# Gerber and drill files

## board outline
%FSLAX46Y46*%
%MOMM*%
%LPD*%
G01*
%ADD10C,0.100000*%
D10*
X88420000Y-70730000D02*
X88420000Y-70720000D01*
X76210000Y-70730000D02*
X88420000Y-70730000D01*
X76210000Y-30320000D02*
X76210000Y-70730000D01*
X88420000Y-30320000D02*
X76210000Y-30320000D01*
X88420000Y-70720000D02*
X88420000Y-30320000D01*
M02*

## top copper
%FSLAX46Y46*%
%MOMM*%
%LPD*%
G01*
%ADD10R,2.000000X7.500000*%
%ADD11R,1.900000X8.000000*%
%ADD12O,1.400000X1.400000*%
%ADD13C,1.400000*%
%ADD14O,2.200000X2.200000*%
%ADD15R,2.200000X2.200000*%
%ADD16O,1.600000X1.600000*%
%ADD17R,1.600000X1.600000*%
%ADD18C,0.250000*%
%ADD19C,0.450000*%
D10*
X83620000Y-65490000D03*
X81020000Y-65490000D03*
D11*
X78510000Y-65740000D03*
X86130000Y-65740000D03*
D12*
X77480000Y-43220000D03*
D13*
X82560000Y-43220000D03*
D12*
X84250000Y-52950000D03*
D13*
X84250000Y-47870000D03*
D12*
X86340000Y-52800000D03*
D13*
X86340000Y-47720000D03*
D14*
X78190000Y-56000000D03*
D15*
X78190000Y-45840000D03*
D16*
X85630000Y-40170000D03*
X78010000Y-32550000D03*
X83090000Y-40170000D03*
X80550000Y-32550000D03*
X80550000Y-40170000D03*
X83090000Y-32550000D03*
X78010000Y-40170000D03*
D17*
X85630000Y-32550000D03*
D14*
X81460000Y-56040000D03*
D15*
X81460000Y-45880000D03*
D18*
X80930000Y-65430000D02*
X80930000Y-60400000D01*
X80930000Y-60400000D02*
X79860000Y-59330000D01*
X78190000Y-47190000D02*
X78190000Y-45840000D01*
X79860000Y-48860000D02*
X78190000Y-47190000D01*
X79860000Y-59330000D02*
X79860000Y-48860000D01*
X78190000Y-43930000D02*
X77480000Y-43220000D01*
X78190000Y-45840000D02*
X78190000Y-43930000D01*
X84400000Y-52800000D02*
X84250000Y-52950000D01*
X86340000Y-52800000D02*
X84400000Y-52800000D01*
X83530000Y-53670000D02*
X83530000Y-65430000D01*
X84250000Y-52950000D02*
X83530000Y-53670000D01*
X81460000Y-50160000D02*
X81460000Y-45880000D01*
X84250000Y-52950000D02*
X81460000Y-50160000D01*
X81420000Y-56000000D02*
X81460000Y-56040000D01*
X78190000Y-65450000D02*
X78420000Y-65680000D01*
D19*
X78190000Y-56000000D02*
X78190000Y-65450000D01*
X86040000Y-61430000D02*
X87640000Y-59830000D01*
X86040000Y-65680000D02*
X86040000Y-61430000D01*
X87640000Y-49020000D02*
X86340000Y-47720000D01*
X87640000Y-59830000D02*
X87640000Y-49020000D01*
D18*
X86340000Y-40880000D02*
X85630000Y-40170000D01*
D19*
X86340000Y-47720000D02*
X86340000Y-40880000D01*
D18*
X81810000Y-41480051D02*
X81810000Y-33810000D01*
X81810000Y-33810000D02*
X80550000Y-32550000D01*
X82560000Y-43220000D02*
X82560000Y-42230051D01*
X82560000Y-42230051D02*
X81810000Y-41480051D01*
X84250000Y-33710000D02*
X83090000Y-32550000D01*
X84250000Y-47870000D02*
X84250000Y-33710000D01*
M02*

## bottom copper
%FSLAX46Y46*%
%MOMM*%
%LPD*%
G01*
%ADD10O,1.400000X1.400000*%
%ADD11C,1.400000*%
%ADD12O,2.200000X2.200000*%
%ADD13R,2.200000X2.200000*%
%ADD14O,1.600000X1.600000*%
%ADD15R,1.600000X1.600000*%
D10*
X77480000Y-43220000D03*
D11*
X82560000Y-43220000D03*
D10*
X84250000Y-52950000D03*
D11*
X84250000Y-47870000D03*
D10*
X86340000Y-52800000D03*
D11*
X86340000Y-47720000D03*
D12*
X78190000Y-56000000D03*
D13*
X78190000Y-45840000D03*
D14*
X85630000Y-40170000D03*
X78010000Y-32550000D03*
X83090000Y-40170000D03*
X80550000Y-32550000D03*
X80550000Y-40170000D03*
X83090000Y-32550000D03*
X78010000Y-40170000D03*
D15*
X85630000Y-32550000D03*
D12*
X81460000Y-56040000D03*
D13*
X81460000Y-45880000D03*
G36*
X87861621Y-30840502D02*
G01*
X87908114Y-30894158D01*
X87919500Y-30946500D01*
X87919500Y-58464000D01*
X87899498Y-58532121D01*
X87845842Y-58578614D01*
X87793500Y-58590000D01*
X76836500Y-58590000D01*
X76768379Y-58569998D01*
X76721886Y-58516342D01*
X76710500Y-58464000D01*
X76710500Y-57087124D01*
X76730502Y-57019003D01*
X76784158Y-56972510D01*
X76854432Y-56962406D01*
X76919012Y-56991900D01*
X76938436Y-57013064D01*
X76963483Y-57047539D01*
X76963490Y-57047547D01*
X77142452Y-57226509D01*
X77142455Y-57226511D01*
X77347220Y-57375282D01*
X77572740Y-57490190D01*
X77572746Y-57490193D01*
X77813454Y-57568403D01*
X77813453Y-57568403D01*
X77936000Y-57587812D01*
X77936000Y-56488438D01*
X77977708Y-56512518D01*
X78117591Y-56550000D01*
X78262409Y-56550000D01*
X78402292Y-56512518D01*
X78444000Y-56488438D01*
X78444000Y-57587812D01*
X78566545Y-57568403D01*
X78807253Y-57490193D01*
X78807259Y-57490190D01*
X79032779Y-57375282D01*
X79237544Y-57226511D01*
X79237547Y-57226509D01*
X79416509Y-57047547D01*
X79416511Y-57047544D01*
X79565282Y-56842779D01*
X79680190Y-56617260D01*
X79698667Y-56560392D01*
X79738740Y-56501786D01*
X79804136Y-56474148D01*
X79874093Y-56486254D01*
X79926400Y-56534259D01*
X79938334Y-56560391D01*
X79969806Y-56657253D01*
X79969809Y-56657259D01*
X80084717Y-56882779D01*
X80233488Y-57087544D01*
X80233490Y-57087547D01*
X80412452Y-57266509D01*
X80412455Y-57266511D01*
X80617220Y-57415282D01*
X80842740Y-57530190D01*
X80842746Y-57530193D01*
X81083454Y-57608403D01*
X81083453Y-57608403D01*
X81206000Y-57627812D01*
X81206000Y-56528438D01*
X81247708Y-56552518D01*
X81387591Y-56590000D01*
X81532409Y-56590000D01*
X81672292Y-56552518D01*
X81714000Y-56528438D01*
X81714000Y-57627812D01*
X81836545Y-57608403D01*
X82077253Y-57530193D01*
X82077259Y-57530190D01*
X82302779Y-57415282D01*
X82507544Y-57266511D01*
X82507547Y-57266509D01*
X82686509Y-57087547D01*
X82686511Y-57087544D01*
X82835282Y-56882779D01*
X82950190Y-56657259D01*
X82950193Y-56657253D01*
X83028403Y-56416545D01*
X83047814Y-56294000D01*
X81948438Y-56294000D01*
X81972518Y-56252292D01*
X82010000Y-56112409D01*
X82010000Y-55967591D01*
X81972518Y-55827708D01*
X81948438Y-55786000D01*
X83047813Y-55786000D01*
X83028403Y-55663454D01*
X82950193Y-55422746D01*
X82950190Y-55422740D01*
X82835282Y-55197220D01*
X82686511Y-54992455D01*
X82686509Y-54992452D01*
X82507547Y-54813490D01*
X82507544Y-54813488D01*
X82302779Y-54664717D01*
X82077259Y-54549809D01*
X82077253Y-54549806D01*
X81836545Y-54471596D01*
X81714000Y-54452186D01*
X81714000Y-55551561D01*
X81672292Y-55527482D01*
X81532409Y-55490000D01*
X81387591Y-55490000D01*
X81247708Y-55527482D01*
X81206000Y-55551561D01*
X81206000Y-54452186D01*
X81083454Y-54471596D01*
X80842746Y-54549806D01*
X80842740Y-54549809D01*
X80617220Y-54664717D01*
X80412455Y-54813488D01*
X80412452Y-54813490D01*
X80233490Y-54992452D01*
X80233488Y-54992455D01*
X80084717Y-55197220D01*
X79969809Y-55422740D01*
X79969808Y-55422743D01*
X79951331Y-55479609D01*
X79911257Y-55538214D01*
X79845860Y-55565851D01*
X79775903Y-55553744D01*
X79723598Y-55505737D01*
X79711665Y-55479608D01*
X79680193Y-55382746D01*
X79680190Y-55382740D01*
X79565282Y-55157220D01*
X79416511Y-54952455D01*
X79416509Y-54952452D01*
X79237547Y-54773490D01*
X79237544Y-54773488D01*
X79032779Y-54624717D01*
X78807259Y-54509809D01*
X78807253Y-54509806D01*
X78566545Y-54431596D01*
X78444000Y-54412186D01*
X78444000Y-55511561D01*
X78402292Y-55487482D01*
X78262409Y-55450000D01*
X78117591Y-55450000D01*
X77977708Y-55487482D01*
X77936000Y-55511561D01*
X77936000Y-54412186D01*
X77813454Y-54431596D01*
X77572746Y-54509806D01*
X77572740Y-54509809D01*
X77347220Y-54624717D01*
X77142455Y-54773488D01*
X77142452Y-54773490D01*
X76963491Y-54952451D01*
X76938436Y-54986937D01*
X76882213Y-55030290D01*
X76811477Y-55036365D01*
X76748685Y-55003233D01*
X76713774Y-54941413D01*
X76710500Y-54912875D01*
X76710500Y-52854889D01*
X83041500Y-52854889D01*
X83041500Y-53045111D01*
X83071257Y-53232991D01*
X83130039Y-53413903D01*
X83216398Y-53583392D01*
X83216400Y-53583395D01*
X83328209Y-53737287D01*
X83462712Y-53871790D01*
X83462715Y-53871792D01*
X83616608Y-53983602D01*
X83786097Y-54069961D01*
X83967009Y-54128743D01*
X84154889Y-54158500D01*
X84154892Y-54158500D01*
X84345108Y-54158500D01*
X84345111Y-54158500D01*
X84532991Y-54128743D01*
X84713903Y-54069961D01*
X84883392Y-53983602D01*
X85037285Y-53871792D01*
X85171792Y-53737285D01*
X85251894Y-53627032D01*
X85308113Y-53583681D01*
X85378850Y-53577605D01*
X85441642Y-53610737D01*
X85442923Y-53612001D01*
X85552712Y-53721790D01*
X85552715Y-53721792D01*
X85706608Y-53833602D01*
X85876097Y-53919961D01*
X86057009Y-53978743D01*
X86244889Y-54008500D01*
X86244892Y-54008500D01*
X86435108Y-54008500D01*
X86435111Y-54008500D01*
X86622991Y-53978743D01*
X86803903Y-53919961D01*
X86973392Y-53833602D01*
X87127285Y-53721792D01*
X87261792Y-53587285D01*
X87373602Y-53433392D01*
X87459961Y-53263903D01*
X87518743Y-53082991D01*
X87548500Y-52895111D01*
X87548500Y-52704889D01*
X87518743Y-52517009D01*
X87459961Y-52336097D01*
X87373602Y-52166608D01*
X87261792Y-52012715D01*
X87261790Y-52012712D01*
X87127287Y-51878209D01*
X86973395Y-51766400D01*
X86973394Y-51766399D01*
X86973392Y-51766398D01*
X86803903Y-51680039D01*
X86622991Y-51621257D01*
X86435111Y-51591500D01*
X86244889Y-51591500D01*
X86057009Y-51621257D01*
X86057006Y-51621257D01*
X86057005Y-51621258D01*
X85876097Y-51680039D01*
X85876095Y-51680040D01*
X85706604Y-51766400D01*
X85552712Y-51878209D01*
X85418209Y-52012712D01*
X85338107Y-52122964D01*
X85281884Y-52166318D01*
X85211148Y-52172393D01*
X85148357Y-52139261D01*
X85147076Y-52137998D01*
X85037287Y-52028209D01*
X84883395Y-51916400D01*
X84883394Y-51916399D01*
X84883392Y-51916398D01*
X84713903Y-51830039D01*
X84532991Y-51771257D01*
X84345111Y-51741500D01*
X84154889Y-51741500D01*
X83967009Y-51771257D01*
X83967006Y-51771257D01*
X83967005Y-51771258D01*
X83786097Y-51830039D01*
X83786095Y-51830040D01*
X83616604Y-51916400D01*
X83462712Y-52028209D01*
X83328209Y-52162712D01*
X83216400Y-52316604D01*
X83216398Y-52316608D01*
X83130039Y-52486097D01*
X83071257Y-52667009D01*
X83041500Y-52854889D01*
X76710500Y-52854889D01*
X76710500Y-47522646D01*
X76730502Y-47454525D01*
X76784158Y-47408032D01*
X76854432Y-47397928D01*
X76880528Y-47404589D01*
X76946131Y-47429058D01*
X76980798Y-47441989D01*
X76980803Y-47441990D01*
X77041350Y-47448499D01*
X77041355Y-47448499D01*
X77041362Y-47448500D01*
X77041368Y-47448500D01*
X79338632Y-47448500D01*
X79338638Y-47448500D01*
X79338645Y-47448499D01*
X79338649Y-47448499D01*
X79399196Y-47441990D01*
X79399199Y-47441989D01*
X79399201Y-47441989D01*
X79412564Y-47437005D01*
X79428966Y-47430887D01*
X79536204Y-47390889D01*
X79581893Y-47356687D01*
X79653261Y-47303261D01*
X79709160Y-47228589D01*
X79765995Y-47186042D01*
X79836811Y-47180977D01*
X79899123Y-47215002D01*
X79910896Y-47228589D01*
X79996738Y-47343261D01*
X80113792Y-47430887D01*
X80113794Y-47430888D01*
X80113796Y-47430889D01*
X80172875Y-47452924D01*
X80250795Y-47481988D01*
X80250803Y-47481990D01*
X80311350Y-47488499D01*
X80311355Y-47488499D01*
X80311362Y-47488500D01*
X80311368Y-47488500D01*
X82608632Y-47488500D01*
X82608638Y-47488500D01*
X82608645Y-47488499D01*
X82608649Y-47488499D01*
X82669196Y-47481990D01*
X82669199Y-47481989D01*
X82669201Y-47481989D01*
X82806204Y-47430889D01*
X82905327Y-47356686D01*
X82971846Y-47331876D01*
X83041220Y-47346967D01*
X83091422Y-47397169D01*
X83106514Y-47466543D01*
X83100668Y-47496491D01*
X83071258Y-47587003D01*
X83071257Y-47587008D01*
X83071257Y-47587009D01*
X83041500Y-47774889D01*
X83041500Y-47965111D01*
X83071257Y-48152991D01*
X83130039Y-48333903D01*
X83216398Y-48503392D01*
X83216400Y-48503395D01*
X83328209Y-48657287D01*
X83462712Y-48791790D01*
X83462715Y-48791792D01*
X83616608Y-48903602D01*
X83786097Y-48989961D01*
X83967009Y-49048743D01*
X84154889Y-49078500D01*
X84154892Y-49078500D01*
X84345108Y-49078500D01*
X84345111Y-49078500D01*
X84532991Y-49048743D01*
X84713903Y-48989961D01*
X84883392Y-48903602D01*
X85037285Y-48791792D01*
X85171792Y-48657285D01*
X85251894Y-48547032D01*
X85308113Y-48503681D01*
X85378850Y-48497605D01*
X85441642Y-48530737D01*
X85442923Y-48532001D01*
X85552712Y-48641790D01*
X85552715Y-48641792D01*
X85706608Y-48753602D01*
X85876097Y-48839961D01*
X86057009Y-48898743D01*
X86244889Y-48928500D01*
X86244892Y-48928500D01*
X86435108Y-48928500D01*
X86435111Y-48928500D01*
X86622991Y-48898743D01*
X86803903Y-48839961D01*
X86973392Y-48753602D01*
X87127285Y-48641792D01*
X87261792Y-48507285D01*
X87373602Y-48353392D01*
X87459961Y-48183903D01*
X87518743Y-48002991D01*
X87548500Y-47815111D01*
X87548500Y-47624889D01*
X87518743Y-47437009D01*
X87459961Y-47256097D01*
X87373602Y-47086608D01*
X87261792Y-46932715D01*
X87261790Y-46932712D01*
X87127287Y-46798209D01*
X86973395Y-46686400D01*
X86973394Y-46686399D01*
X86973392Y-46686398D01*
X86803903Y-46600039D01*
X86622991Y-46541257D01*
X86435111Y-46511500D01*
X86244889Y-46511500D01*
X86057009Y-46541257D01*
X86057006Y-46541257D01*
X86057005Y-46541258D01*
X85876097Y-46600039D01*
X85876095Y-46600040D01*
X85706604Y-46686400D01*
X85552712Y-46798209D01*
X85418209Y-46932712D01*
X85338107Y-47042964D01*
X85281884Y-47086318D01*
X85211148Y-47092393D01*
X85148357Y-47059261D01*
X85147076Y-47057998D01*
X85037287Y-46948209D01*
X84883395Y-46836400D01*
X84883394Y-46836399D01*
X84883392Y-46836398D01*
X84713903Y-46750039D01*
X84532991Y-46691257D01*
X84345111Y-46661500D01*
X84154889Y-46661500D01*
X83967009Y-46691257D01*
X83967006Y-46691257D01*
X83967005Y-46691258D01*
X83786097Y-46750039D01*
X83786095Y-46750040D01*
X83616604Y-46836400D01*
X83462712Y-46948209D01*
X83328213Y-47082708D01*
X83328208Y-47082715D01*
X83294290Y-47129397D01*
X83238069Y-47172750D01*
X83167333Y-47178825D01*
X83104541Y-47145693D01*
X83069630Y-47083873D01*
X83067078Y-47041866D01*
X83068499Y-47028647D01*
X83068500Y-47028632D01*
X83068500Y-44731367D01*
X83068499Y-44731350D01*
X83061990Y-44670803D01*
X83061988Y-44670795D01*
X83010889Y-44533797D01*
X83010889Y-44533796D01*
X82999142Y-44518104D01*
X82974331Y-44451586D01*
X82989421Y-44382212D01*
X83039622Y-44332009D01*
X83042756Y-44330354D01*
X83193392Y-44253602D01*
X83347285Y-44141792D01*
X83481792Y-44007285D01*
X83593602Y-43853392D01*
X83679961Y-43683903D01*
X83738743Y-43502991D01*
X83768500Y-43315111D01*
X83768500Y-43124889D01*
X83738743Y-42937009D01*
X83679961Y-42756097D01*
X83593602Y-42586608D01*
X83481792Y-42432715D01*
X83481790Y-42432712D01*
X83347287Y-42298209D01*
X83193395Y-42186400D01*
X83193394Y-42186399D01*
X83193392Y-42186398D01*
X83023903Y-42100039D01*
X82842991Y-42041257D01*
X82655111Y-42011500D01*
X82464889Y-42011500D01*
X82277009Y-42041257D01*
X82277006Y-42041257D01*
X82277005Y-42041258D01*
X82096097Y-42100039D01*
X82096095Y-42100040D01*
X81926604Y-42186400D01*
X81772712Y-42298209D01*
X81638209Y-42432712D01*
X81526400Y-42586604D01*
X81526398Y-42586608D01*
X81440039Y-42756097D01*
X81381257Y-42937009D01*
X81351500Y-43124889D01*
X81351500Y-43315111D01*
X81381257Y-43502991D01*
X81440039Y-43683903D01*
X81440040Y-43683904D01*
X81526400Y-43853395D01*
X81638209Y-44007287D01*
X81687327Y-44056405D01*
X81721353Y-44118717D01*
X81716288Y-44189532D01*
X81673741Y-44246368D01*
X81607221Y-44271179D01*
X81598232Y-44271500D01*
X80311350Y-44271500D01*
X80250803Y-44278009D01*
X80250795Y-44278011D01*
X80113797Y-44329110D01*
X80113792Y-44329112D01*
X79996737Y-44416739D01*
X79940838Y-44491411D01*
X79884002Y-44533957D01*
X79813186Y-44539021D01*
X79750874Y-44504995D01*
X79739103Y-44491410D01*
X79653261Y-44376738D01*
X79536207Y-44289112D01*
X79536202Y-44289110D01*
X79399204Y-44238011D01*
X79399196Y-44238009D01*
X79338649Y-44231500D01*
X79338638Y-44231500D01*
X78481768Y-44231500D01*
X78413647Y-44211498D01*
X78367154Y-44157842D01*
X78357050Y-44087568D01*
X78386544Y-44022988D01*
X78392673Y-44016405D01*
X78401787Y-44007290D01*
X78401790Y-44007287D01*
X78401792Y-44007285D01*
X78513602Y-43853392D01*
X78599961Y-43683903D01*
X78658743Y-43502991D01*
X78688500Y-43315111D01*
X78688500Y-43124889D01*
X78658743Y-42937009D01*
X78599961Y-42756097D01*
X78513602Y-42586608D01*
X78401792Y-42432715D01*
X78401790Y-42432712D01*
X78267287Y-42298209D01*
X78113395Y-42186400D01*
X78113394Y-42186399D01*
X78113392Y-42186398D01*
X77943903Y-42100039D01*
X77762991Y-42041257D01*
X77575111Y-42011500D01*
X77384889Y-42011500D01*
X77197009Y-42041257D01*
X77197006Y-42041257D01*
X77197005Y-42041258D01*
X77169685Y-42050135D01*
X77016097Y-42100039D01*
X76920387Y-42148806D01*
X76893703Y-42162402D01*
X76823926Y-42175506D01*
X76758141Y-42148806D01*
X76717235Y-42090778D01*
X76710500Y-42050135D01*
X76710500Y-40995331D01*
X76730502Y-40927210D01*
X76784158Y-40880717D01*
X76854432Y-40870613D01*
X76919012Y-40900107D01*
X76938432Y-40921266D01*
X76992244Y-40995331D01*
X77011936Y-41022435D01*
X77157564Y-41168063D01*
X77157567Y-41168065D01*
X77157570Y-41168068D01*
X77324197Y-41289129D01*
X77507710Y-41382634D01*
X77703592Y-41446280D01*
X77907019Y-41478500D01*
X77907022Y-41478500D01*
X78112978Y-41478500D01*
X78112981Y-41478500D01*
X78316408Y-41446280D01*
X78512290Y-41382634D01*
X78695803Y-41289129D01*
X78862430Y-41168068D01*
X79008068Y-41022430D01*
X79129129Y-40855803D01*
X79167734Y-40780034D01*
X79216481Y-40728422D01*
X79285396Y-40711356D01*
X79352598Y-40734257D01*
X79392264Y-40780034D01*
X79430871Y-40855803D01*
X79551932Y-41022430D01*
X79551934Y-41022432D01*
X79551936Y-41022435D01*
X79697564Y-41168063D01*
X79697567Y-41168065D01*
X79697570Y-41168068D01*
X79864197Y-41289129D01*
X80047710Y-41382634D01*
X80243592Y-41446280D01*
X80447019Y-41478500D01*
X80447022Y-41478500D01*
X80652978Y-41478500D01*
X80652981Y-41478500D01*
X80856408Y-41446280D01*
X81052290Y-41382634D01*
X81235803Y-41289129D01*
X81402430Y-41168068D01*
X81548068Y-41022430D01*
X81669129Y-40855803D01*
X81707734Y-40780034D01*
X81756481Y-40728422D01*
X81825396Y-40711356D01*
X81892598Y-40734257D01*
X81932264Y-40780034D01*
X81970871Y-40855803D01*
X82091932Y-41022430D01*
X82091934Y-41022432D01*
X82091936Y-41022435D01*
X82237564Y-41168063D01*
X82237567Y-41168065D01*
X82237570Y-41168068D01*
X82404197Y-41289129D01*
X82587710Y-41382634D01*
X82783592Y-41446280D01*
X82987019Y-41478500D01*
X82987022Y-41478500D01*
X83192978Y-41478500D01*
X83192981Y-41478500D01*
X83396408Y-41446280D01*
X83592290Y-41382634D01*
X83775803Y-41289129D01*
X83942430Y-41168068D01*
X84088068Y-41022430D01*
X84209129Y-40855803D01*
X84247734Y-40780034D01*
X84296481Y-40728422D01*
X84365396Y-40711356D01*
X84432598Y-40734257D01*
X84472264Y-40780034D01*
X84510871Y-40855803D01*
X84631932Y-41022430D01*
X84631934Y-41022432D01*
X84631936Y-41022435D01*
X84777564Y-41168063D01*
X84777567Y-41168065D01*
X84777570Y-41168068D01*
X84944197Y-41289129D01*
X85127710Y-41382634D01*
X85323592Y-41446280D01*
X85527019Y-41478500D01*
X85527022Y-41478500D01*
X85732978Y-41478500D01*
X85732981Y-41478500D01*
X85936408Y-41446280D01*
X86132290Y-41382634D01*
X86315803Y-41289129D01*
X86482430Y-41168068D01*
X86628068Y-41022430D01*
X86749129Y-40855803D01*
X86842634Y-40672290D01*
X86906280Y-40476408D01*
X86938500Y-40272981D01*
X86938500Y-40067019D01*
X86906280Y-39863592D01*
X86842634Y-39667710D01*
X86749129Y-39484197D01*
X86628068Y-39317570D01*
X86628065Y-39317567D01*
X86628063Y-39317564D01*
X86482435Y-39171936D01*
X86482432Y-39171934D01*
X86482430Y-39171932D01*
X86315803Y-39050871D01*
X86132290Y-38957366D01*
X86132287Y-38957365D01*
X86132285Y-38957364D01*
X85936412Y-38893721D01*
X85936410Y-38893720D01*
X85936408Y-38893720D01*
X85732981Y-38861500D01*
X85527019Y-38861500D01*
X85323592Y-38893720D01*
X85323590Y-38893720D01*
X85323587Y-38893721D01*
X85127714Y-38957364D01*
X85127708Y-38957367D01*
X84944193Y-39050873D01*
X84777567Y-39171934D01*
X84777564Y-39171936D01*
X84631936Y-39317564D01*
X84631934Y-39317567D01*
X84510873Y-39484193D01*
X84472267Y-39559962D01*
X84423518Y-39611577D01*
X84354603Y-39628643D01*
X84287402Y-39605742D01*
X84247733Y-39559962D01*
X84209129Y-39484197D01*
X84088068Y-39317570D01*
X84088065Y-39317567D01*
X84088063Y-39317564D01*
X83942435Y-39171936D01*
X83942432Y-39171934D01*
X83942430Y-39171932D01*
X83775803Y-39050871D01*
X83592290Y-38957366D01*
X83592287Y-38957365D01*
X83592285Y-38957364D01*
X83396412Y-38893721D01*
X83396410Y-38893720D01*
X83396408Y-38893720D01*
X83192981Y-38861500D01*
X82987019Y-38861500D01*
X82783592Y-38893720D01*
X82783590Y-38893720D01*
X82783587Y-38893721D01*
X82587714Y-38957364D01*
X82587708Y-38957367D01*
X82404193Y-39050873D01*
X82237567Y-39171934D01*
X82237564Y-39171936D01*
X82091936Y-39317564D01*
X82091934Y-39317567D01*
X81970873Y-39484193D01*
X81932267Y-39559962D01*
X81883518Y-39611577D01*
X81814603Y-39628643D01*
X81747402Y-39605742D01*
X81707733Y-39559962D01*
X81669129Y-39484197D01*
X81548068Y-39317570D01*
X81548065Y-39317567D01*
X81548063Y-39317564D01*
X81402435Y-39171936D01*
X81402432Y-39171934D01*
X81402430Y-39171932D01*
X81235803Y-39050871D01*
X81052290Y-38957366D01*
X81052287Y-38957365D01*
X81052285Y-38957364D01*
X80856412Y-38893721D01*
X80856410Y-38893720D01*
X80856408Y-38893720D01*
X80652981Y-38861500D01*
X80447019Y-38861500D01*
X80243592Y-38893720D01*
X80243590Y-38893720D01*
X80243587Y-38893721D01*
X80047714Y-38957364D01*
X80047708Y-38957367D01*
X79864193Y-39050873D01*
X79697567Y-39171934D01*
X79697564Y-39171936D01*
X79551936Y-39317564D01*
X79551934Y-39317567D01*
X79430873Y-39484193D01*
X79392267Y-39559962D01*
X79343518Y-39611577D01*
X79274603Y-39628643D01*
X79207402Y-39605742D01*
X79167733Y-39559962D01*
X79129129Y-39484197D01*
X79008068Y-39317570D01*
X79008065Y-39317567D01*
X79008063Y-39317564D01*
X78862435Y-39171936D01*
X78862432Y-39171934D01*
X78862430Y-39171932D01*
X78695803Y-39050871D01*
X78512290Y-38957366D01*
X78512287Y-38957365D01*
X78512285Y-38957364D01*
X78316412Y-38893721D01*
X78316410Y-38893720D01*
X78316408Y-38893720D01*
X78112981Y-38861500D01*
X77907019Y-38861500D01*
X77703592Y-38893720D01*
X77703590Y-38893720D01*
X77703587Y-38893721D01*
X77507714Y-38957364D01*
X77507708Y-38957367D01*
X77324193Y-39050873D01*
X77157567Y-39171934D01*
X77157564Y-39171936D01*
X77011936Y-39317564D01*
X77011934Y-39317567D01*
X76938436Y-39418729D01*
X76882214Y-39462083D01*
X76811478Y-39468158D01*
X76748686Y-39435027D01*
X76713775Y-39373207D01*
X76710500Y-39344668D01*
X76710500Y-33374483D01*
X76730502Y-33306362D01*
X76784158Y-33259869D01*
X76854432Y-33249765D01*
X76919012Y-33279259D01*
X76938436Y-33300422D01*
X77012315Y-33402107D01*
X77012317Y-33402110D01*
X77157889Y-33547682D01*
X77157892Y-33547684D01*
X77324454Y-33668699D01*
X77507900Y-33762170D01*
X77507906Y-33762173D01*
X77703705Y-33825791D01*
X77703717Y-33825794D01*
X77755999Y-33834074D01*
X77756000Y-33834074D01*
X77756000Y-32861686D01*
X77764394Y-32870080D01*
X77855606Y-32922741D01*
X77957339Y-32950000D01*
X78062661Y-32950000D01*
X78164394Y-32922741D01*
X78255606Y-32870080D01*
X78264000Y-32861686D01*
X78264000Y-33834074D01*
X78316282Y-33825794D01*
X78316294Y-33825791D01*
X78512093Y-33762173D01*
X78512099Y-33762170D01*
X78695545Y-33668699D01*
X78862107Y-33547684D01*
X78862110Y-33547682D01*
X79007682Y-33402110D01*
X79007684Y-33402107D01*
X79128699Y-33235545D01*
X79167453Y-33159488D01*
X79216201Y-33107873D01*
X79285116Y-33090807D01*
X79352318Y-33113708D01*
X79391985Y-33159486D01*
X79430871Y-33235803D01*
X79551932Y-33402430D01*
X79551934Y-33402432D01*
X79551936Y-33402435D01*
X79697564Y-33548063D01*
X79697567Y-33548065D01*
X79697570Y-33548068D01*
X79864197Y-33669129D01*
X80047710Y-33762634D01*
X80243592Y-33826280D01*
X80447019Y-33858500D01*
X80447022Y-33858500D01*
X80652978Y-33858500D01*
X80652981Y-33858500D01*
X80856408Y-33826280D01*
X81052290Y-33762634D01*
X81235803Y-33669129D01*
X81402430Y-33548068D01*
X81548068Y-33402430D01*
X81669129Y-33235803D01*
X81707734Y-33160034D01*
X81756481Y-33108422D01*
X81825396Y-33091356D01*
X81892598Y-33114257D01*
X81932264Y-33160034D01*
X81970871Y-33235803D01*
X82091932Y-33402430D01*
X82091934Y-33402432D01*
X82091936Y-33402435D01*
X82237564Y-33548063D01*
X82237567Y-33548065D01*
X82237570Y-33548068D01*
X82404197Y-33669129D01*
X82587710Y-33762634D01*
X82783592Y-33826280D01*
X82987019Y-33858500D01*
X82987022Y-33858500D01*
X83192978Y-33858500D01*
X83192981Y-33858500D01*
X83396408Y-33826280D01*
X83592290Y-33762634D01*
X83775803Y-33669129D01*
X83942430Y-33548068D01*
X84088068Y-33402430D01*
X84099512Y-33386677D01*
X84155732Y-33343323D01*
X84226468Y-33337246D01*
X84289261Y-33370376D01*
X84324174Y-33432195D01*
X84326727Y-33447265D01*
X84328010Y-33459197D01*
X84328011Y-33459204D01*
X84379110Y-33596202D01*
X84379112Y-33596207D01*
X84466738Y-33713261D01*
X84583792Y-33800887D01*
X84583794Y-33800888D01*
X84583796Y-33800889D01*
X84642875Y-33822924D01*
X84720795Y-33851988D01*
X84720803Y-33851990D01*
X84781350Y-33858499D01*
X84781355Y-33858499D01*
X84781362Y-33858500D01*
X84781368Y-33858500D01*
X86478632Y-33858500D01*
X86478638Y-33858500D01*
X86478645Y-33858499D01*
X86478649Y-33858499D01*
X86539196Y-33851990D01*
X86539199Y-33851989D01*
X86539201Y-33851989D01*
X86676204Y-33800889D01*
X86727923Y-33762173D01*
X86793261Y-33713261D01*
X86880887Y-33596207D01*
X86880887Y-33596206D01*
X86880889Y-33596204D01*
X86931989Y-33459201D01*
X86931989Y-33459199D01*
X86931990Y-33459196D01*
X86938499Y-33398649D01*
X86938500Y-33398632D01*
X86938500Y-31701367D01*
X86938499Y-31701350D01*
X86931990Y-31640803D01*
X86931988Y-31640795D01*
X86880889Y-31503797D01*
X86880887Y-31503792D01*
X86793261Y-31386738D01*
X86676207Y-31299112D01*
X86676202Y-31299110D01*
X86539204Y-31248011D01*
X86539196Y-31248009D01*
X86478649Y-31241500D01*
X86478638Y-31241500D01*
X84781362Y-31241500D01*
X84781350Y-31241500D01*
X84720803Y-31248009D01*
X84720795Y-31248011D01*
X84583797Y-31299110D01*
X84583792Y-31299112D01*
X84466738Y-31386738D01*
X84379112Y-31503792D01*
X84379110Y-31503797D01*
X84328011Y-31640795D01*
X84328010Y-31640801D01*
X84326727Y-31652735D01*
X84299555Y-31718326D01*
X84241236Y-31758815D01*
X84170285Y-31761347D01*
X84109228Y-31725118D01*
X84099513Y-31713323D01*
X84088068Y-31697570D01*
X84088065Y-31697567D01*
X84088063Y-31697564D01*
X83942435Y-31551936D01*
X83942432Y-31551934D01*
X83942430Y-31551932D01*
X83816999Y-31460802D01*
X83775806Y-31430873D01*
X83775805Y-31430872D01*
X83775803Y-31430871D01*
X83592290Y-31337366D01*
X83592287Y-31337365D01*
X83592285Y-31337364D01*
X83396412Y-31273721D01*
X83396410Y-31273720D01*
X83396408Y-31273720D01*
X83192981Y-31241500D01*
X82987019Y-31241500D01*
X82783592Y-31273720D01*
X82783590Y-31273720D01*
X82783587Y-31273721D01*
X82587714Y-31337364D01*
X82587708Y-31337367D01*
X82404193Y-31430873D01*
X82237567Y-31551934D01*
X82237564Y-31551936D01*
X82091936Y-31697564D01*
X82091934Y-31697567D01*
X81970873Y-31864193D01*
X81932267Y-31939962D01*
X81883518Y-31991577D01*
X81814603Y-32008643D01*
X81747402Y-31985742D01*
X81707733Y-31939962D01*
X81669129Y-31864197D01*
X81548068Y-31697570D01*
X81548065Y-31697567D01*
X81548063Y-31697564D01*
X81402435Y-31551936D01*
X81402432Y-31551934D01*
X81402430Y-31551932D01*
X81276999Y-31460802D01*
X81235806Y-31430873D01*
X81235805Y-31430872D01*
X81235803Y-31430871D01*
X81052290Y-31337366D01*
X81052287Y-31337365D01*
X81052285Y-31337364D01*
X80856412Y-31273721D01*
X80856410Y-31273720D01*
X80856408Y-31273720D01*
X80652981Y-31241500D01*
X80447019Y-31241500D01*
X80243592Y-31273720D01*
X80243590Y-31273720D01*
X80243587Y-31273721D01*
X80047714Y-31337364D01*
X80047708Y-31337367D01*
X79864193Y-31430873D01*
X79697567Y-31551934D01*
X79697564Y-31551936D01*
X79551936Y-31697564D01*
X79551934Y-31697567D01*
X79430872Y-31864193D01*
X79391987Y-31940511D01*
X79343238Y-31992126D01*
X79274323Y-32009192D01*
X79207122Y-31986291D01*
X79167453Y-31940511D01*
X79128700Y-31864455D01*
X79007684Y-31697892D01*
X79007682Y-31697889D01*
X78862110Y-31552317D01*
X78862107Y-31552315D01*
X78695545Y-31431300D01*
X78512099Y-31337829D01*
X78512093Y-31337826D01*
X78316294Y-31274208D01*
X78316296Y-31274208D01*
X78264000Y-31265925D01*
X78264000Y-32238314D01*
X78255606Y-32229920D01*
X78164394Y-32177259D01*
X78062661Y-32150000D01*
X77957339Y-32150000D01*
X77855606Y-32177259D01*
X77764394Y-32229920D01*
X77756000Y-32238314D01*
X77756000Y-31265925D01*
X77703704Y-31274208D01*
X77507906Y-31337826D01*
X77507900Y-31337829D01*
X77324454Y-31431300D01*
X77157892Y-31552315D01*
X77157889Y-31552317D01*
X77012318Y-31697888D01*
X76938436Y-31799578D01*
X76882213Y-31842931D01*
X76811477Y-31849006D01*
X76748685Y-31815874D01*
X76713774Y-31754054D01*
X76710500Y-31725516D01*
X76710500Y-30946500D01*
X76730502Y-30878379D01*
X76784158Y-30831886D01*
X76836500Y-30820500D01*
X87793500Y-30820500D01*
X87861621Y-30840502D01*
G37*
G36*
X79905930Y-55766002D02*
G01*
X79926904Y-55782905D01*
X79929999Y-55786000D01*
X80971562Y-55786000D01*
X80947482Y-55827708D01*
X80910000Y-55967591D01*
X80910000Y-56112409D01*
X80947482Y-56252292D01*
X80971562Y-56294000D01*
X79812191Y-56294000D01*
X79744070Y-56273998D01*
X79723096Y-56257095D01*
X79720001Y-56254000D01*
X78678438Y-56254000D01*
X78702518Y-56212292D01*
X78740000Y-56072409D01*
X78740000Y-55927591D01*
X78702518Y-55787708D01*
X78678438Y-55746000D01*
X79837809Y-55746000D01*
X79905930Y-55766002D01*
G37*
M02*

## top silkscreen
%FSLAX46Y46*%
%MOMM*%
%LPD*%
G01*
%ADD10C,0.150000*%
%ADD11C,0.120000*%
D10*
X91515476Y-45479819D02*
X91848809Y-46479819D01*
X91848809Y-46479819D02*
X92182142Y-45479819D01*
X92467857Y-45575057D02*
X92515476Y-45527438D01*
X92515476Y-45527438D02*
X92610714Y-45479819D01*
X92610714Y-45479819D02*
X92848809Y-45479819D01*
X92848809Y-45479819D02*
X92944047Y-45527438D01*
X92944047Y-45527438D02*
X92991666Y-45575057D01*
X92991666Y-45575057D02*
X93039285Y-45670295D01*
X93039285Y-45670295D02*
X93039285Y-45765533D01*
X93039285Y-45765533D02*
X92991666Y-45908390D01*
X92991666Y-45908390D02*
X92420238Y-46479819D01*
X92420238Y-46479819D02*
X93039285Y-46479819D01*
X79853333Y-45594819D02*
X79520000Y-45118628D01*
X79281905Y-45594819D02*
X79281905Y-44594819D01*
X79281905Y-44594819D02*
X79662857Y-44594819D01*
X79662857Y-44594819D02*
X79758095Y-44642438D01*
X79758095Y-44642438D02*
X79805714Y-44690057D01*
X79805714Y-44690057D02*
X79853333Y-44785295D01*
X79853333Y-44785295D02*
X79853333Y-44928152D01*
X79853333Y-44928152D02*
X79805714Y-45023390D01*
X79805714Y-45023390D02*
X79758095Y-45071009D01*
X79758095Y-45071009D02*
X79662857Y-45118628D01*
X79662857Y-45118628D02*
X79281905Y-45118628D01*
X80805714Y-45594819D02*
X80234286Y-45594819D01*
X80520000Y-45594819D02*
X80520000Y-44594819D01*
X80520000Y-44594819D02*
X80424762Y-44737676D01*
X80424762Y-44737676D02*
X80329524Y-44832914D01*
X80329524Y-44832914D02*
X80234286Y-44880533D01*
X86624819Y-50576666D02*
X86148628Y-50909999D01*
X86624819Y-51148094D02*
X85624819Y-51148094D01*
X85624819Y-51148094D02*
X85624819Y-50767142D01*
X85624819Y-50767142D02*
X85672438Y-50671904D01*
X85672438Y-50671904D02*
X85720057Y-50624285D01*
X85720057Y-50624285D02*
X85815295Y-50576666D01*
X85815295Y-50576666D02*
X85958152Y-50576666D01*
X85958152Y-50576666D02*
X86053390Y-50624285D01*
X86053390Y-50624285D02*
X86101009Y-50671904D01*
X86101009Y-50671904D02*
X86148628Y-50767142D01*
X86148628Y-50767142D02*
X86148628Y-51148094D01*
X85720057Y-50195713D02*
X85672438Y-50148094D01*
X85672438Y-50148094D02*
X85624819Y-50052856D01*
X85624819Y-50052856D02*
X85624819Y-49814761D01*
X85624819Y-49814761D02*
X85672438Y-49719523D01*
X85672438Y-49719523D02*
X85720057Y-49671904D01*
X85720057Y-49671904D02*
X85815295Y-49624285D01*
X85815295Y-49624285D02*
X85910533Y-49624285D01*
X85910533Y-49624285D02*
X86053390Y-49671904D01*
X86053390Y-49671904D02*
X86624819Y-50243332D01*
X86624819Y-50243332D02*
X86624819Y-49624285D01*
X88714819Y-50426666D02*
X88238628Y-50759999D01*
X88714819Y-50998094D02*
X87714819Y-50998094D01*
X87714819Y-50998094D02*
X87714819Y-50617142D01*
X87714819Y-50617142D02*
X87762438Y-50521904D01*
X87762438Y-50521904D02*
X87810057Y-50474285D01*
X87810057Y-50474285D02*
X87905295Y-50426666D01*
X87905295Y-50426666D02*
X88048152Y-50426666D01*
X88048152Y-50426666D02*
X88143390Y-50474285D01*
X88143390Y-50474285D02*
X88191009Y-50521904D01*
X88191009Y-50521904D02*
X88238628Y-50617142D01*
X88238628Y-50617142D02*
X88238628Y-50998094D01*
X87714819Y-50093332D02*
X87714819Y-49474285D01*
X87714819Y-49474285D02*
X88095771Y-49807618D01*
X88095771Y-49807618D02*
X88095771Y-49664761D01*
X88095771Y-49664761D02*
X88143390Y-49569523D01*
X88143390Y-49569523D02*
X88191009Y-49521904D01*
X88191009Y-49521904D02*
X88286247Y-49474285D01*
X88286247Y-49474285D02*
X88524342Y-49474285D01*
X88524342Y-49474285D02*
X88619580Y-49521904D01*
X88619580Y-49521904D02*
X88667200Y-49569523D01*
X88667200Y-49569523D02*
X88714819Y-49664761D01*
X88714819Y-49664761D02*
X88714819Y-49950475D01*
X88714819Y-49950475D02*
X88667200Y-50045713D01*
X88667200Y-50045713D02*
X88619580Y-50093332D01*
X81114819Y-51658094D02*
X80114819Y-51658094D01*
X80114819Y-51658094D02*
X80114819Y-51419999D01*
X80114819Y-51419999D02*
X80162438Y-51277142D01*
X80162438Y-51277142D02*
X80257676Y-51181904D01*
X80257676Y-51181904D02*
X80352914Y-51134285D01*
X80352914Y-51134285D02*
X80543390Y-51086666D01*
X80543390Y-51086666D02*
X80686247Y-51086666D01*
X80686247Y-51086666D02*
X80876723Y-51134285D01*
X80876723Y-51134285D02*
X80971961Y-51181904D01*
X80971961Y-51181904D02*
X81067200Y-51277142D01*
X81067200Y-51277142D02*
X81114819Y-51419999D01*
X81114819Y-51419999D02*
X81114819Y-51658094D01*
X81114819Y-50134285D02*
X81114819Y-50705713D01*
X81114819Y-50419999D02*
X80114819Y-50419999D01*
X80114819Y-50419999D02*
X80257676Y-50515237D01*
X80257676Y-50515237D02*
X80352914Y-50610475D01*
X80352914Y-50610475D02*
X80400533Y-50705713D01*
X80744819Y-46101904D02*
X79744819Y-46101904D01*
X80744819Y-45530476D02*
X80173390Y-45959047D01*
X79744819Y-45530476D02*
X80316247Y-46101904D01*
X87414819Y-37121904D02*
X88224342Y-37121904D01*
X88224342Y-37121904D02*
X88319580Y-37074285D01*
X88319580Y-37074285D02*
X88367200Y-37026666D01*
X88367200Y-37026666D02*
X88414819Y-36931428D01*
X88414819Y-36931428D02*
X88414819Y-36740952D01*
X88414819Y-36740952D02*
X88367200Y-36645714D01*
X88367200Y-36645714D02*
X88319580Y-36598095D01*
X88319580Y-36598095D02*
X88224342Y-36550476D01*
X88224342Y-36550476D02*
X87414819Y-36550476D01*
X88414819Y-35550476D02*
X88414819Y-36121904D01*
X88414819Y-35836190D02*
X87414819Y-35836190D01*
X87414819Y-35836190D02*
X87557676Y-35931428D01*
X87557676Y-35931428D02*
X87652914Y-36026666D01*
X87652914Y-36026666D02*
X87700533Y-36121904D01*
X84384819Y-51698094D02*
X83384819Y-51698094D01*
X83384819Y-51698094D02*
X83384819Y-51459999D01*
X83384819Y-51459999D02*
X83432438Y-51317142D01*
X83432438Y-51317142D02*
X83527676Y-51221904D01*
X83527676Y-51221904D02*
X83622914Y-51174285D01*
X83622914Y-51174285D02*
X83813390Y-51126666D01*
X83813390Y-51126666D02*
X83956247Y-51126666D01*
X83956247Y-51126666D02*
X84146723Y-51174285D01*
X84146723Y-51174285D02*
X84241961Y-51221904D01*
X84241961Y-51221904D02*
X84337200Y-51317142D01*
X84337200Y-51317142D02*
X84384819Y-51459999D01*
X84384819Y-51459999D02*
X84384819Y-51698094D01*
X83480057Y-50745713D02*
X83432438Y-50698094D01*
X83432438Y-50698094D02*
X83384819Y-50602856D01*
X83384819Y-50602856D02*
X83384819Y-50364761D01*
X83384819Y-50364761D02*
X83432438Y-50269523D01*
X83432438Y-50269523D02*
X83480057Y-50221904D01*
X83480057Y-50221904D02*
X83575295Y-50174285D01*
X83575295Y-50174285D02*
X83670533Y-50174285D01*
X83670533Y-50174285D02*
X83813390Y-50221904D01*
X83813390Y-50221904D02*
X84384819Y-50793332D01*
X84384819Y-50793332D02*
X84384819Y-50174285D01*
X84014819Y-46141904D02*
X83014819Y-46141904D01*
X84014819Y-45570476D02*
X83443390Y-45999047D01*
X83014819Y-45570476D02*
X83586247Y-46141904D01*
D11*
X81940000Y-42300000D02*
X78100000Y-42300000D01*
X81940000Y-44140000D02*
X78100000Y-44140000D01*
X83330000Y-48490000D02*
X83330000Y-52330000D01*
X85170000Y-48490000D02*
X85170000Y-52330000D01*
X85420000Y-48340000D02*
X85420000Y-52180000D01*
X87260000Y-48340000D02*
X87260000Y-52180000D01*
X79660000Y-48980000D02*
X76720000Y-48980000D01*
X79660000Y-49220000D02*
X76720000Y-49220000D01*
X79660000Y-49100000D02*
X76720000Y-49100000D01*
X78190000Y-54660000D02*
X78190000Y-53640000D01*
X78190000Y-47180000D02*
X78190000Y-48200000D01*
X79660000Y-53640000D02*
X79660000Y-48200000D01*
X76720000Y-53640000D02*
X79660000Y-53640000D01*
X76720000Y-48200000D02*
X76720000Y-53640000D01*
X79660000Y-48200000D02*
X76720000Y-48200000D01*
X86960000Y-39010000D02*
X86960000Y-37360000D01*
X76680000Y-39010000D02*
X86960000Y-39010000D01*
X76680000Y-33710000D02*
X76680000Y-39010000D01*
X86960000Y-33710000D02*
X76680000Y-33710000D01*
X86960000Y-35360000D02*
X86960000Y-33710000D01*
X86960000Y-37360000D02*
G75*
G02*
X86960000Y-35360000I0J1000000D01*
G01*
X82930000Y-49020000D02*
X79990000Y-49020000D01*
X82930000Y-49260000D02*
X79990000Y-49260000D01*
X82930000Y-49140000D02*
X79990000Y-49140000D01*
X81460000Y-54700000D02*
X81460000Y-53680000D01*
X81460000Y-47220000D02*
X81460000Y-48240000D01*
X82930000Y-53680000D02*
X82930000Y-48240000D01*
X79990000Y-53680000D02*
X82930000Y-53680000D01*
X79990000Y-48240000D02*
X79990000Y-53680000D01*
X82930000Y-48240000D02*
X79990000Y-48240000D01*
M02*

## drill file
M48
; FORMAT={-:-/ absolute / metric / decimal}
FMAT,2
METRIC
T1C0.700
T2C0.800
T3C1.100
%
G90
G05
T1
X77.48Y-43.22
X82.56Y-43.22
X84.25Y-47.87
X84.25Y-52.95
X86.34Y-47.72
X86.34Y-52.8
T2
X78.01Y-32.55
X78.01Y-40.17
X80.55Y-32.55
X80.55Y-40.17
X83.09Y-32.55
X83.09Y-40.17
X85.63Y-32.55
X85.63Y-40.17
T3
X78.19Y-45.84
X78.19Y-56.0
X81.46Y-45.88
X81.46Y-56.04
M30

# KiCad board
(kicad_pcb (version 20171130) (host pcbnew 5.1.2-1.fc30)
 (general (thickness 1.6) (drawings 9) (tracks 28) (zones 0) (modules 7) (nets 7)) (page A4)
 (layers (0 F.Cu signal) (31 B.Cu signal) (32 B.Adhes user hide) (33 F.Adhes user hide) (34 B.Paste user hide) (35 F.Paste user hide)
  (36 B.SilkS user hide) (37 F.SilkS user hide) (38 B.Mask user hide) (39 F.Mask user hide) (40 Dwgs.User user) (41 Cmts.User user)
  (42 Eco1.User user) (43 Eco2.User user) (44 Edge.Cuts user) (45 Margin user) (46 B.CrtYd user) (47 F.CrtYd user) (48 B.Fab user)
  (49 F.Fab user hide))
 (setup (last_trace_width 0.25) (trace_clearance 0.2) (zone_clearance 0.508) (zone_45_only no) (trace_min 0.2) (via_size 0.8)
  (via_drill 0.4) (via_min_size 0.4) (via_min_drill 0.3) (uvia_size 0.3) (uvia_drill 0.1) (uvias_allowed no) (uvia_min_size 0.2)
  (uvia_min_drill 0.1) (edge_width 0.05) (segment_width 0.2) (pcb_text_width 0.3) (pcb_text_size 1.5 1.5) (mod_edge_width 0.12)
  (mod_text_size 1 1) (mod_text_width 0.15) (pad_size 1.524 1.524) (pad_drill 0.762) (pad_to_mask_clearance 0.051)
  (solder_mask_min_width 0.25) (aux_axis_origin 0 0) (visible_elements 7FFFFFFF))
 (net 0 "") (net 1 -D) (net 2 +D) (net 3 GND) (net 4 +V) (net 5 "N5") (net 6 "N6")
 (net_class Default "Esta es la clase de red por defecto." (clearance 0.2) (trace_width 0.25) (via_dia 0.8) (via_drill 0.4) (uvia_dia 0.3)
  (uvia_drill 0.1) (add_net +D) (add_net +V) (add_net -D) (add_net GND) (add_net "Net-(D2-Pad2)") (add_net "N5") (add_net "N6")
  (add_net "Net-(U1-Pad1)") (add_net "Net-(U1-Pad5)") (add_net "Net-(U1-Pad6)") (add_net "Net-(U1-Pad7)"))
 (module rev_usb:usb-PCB (layer F.Cu) (at 82.32 70.64)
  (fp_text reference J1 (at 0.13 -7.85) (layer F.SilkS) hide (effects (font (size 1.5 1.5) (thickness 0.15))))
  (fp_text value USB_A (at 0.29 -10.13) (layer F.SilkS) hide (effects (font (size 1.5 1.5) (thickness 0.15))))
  (pad 2 connect rect (at 1.3 -5.15) (size 2 7.5) (layers F.Cu F.Mask) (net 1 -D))
  (pad 3 connect rect (at -1.3 -5.15) (size 2 7.5) (layers F.Cu F.Mask) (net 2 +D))
  (pad 4 connect rect (at -3.81 -4.9) (size 1.9 8) (layers F.Cu F.Mask) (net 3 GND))
  (pad 1 connect rect (at 3.81 -4.9) (size 1.9 8) (layers F.Cu F.Mask) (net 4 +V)))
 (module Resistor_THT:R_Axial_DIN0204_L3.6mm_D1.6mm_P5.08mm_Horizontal (layer F.Cu) (at 82.56 43.22 180)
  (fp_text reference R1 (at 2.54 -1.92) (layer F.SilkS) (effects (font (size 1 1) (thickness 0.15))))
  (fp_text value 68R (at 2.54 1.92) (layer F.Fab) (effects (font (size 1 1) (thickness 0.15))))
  (fp_line (start 0.62 0.92) (end 4.46 0.92) (layer F.SilkS) (width 0.12))
  (fp_line (start 0.62 -0.92) (end 4.46 -0.92) (layer F.SilkS) (width 0.12))
  (pad 2 thru_hole oval (at 5.08 0 180) (size 1.4 1.4) (drill 0.7) (layers *.Cu *.Mask) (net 2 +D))
  (pad 1 thru_hole circle (at 0 0 180) (size 1.4 1.4) (drill 0.7) (layers *.Cu *.Mask) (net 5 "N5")))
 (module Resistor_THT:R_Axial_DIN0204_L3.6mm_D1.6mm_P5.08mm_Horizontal (layer F.Cu) (at 84.25 47.87 270)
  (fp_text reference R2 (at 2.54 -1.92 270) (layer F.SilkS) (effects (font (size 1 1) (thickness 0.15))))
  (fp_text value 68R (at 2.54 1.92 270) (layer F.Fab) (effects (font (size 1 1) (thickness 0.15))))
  (fp_line (start 0.62 0.92) (end 4.46 0.92) (layer F.SilkS) (width 0.12))
  (fp_line (start 0.62 -0.92) (end 4.46 -0.92) (layer F.SilkS) (width 0.12))
  (pad 2 thru_hole oval (at 5.08 0 270) (size 1.4 1.4) (drill 0.7) (layers *.Cu *.Mask) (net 1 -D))
  (pad 1 thru_hole circle (at 0 0 270) (size 1.4 1.4) (drill 0.7) (layers *.Cu *.Mask) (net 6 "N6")))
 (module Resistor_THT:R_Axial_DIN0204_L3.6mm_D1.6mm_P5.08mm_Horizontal (layer F.Cu) (at 86.34 47.72 270)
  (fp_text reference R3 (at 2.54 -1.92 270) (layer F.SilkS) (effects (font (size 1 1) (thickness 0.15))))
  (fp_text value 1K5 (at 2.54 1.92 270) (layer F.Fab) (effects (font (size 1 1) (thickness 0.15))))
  (fp_line (start 0.62 0.92) (end 4.46 0.92) (layer F.SilkS) (width 0.12))
  (fp_line (start 0.62 -0.92) (end 4.46 -0.92) (layer F.SilkS) (width 0.12))
  (pad 2 thru_hole oval (at 5.08 0 270) (size 1.4 1.4) (drill 0.7) (layers *.Cu *.Mask) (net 1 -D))
  (pad 1 thru_hole circle (at 0 0 270) (size 1.4 1.4) (drill 0.7) (layers *.Cu *.Mask) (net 4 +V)))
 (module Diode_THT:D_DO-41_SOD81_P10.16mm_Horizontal (layer F.Cu) (at 78.19 45.84 270)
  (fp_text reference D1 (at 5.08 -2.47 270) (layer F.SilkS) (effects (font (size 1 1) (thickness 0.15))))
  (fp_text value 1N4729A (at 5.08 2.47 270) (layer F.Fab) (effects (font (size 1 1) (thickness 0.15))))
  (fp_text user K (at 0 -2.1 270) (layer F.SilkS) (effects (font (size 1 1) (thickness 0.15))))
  (fp_line (start 3.14 -1.47) (end 3.14 1.47) (layer F.SilkS) (width 0.12))
  (fp_line (start 3.38 -1.47) (end 3.38 1.47) (layer F.SilkS) (width 0.12))
  (fp_line (start 3.26 -1.47) (end 3.26 1.47) (layer F.SilkS) (width 0.12))
  (fp_line (start 8.82 0) (end 7.8 0) (layer F.SilkS) (width 0.12))
  (fp_line (start 1.34 0) (end 2.36 0) (layer F.SilkS) (width 0.12))
  (fp_line (start 7.8 -1.47) (end 2.36 -1.47) (layer F.SilkS) (width 0.12))
  (fp_line (start 7.8 1.47) (end 7.8 -1.47) (layer F.SilkS) (width 0.12))
  (fp_line (start 2.36 1.47) (end 7.8 1.47) (layer F.SilkS) (width 0.12))
  (fp_line (start 2.36 -1.47) (end 2.36 1.47) (layer F.SilkS) (width 0.12))
  (pad 2 thru_hole oval (at 10.16 0 270) (size 2.2 2.2) (drill 1.1) (layers *.Cu *.Mask) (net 3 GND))
  (pad 1 thru_hole rect (at 0 0 270) (size 2.2 2.2) (drill 1.1) (layers *.Cu *.Mask) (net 2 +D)))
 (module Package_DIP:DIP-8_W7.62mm (layer F.Cu) (at 85.63 32.55 270)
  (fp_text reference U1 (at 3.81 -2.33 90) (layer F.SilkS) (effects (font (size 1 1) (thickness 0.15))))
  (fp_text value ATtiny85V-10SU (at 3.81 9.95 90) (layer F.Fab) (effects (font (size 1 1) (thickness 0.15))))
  (fp_line (start 6.46 -1.33) (end 4.81 -1.33) (layer F.SilkS) (width 0.12))
  (fp_line (start 6.46 8.95) (end 6.46 -1.33) (layer F.SilkS) (width 0.12))
  (fp_line (start 1.16 8.95) (end 6.46 8.95) (layer F.SilkS) (width 0.12))
  (fp_line (start 1.16 -1.33) (end 1.16 8.95) (layer F.SilkS) (width 0.12))
  (fp_line (start 2.81 -1.33) (end 1.16 -1.33) (layer F.SilkS) (width 0.12))
  (fp_arc (start 3.81 -1.33) (end 2.81 -1.33) (angle -180) (layer F.SilkS) (width 0.12))
  (pad 8 thru_hole oval (at 7.62 0 270) (size 1.6 1.6) (drill 0.8) (layers *.Cu *.Mask) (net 4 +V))
  (pad 4 thru_hole oval (at 0 7.62 270) (size 1.6 1.6) (drill 0.8) (layers *.Cu *.Mask) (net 3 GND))
  (pad 7 thru_hole oval (at 7.62 2.54 270) (size 1.6 1.6) (drill 0.8) (layers *.Cu *.Mask))
  (pad 3 thru_hole oval (at 0 5.08 270) (size 1.6 1.6) (drill 0.8) (layers *.Cu *.Mask) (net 5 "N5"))
  (pad 6 thru_hole oval (at 7.62 5.08 270) (size 1.6 1.6) (drill 0.8) (layers *.Cu *.Mask))
  (pad 2 thru_hole oval (at 0 2.54 270) (size 1.6 1.6) (drill 0.8) (layers *.Cu *.Mask) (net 6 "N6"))
  (pad 5 thru_hole oval (at 7.62 7.62 270) (size 1.6 1.6) (drill 0.8) (layers *.Cu *.Mask))
  (pad 1 thru_hole rect (at 0 0 270) (size 1.6 1.6) (drill 0.8) (layers *.Cu *.Mask)))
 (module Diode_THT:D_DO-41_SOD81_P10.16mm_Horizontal (layer F.Cu) (at 81.46 45.88 270)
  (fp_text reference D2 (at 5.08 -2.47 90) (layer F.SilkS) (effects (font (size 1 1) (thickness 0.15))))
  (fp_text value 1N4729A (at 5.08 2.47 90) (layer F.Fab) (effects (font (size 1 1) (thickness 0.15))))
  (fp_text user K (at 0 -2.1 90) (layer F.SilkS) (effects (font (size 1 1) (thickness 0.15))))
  (fp_line (start 3.14 -1.47) (end 3.14 1.47) (layer F.SilkS) (width 0.12))
  (fp_line (start 3.38 -1.47) (end 3.38 1.47) (layer F.SilkS) (width 0.12))
  (fp_line (start 3.26 -1.47) (end 3.26 1.47) (layer F.SilkS) (width 0.12))
  (fp_line (start 8.82 0) (end 7.8 0) (layer F.SilkS) (width 0.12))
  (fp_line (start 1.34 0) (end 2.36 0) (layer F.SilkS) (width 0.12))
  (fp_line (start 7.8 -1.47) (end 2.36 -1.47) (layer F.SilkS) (width 0.12))
  (fp_line (start 7.8 1.47) (end 7.8 -1.47) (layer F.SilkS) (width 0.12))
  (fp_line (start 2.36 1.47) (end 7.8 1.47) (layer F.SilkS) (width 0.12))
  (fp_line (start 2.36 -1.47) (end 2.36 1.47) (layer F.SilkS) (width 0.12))
  (pad 2 thru_hole oval (at 10.16 0 270) (size 2.2 2.2) (drill 1.1) (layers *.Cu *.Mask) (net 3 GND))
  (pad 1 thru_hole rect (at 0 0 270) (size 2.2 2.2) (drill 1.1) (layers *.Cu *.Mask) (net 1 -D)))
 (gr_line (start 88.42 70.73) (end 88.42 70.72) (layer Edge.Cuts) (width 0.1))
 (gr_line (start 76.21 70.73) (end 88.42 70.73) (layer Edge.Cuts) (width 0.1))
 (gr_line (start 76.21 30.32) (end 76.21 70.73) (layer Edge.Cuts) (width 0.1))
 (gr_line (start 88.42 30.32) (end 76.21 30.32) (layer Edge.Cuts) (width 0.1))
 (gr_line (start 88.42 70.72) (end 88.42 30.32) (layer Edge.Cuts) (width 0.1))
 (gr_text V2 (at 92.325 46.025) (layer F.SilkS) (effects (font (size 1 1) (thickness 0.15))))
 (segment (start 80.93 65.43) (end 80.93 60.4) (width 0.25) (layer F.Cu) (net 2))
 (segment (start 80.93 60.4) (end 79.86 59.33) (width 0.25) (layer F.Cu) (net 2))
 (segment (start 78.19 47.19) (end 78.19 45.84) (width 0.25) (layer F.Cu) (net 2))
 (segment (start 79.86 48.86) (end 78.19 47.19) (width 0.25) (layer F.Cu) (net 2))
 (segment (start 79.86 59.33) (end 79.86 48.86) (width 0.25) (layer F.Cu) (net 2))
 (segment (start 78.19 43.93) (end 77.48 43.22) (width 0.25) (layer F.Cu) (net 2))
 (segment (start 78.19 45.84) (end 78.19 43.93) (width 0.25) (layer F.Cu) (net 2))
 (segment (start 84.4 52.8) (end 84.25 52.95) (width 0.25) (layer F.Cu) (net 1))
 (segment (start 86.34 52.8) (end 84.4 52.8) (width 0.25) (layer F.Cu) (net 1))
 (segment (start 83.53 53.67) (end 83.53 65.43) (width 0.25) (layer F.Cu) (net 1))
 (segment (start 84.25 52.95) (end 83.53 53.67) (width 0.25) (layer F.Cu) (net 1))
 (segment (start 81.46 50.16) (end 81.46 45.88) (width 0.25) (layer F.Cu) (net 1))
 (segment (start 84.25 52.95) (end 81.46 50.16) (width 0.25) (layer F.Cu) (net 1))
 (segment (start 81.42 56) (end 81.46 56.04) (width 0.25) (layer F.Cu) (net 3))
 (segment (start 78.19 65.45) (end 78.42 65.68) (width 0.25) (layer F.Cu) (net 3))
 (segment (start 78.19 56) (end 78.19 65.45) (width 0.45) (layer F.Cu) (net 3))
 (segment (start 86.04 61.43) (end 87.64 59.83) (width 0.45) (layer F.Cu) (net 4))
 (segment (start 86.04 65.68) (end 86.04 61.43) (width 0.45) (layer F.Cu) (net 4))
 (segment (start 87.64 49.02) (end 86.34 47.72) (width 0.45) (layer F.Cu) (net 4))
 (segment (start 87.64 59.83) (end 87.64 49.02) (width 0.45) (layer F.Cu) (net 4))
 (segment (start 86.34 40.88) (end 85.63 40.17) (width 0.25) (layer F.Cu) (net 4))
 (segment (start 86.34 47.72) (end 86.34 40.88) (width 0.45) (layer F.Cu) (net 4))
 (segment (start 81.81 41.480051) (end 81.81 33.81) (width 0.25) (layer F.Cu) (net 5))
 (segment (start 81.81 33.81) (end 80.55 32.55) (width 0.25) (layer F.Cu) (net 5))
 (segment (start 82.56 43.22) (end 82.56 42.230051) (width 0.25) (layer F.Cu) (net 5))
 (segment (start 82.56 42.230051) (end 81.81 41.480051) (width 0.25) (layer F.Cu) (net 5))
 (segment (start 84.25 33.71) (end 83.09 32.55) (width 0.25) (layer F.Cu) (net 6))
 (segment (start 84.25 47.87) (end 84.25 33.71) (width 0.25) (layer F.Cu) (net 6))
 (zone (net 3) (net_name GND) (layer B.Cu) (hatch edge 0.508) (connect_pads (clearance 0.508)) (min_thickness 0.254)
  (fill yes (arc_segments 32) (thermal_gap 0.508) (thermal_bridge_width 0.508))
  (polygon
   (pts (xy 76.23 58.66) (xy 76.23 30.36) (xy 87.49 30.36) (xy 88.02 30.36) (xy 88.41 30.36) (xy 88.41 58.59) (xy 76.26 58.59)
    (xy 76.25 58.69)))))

